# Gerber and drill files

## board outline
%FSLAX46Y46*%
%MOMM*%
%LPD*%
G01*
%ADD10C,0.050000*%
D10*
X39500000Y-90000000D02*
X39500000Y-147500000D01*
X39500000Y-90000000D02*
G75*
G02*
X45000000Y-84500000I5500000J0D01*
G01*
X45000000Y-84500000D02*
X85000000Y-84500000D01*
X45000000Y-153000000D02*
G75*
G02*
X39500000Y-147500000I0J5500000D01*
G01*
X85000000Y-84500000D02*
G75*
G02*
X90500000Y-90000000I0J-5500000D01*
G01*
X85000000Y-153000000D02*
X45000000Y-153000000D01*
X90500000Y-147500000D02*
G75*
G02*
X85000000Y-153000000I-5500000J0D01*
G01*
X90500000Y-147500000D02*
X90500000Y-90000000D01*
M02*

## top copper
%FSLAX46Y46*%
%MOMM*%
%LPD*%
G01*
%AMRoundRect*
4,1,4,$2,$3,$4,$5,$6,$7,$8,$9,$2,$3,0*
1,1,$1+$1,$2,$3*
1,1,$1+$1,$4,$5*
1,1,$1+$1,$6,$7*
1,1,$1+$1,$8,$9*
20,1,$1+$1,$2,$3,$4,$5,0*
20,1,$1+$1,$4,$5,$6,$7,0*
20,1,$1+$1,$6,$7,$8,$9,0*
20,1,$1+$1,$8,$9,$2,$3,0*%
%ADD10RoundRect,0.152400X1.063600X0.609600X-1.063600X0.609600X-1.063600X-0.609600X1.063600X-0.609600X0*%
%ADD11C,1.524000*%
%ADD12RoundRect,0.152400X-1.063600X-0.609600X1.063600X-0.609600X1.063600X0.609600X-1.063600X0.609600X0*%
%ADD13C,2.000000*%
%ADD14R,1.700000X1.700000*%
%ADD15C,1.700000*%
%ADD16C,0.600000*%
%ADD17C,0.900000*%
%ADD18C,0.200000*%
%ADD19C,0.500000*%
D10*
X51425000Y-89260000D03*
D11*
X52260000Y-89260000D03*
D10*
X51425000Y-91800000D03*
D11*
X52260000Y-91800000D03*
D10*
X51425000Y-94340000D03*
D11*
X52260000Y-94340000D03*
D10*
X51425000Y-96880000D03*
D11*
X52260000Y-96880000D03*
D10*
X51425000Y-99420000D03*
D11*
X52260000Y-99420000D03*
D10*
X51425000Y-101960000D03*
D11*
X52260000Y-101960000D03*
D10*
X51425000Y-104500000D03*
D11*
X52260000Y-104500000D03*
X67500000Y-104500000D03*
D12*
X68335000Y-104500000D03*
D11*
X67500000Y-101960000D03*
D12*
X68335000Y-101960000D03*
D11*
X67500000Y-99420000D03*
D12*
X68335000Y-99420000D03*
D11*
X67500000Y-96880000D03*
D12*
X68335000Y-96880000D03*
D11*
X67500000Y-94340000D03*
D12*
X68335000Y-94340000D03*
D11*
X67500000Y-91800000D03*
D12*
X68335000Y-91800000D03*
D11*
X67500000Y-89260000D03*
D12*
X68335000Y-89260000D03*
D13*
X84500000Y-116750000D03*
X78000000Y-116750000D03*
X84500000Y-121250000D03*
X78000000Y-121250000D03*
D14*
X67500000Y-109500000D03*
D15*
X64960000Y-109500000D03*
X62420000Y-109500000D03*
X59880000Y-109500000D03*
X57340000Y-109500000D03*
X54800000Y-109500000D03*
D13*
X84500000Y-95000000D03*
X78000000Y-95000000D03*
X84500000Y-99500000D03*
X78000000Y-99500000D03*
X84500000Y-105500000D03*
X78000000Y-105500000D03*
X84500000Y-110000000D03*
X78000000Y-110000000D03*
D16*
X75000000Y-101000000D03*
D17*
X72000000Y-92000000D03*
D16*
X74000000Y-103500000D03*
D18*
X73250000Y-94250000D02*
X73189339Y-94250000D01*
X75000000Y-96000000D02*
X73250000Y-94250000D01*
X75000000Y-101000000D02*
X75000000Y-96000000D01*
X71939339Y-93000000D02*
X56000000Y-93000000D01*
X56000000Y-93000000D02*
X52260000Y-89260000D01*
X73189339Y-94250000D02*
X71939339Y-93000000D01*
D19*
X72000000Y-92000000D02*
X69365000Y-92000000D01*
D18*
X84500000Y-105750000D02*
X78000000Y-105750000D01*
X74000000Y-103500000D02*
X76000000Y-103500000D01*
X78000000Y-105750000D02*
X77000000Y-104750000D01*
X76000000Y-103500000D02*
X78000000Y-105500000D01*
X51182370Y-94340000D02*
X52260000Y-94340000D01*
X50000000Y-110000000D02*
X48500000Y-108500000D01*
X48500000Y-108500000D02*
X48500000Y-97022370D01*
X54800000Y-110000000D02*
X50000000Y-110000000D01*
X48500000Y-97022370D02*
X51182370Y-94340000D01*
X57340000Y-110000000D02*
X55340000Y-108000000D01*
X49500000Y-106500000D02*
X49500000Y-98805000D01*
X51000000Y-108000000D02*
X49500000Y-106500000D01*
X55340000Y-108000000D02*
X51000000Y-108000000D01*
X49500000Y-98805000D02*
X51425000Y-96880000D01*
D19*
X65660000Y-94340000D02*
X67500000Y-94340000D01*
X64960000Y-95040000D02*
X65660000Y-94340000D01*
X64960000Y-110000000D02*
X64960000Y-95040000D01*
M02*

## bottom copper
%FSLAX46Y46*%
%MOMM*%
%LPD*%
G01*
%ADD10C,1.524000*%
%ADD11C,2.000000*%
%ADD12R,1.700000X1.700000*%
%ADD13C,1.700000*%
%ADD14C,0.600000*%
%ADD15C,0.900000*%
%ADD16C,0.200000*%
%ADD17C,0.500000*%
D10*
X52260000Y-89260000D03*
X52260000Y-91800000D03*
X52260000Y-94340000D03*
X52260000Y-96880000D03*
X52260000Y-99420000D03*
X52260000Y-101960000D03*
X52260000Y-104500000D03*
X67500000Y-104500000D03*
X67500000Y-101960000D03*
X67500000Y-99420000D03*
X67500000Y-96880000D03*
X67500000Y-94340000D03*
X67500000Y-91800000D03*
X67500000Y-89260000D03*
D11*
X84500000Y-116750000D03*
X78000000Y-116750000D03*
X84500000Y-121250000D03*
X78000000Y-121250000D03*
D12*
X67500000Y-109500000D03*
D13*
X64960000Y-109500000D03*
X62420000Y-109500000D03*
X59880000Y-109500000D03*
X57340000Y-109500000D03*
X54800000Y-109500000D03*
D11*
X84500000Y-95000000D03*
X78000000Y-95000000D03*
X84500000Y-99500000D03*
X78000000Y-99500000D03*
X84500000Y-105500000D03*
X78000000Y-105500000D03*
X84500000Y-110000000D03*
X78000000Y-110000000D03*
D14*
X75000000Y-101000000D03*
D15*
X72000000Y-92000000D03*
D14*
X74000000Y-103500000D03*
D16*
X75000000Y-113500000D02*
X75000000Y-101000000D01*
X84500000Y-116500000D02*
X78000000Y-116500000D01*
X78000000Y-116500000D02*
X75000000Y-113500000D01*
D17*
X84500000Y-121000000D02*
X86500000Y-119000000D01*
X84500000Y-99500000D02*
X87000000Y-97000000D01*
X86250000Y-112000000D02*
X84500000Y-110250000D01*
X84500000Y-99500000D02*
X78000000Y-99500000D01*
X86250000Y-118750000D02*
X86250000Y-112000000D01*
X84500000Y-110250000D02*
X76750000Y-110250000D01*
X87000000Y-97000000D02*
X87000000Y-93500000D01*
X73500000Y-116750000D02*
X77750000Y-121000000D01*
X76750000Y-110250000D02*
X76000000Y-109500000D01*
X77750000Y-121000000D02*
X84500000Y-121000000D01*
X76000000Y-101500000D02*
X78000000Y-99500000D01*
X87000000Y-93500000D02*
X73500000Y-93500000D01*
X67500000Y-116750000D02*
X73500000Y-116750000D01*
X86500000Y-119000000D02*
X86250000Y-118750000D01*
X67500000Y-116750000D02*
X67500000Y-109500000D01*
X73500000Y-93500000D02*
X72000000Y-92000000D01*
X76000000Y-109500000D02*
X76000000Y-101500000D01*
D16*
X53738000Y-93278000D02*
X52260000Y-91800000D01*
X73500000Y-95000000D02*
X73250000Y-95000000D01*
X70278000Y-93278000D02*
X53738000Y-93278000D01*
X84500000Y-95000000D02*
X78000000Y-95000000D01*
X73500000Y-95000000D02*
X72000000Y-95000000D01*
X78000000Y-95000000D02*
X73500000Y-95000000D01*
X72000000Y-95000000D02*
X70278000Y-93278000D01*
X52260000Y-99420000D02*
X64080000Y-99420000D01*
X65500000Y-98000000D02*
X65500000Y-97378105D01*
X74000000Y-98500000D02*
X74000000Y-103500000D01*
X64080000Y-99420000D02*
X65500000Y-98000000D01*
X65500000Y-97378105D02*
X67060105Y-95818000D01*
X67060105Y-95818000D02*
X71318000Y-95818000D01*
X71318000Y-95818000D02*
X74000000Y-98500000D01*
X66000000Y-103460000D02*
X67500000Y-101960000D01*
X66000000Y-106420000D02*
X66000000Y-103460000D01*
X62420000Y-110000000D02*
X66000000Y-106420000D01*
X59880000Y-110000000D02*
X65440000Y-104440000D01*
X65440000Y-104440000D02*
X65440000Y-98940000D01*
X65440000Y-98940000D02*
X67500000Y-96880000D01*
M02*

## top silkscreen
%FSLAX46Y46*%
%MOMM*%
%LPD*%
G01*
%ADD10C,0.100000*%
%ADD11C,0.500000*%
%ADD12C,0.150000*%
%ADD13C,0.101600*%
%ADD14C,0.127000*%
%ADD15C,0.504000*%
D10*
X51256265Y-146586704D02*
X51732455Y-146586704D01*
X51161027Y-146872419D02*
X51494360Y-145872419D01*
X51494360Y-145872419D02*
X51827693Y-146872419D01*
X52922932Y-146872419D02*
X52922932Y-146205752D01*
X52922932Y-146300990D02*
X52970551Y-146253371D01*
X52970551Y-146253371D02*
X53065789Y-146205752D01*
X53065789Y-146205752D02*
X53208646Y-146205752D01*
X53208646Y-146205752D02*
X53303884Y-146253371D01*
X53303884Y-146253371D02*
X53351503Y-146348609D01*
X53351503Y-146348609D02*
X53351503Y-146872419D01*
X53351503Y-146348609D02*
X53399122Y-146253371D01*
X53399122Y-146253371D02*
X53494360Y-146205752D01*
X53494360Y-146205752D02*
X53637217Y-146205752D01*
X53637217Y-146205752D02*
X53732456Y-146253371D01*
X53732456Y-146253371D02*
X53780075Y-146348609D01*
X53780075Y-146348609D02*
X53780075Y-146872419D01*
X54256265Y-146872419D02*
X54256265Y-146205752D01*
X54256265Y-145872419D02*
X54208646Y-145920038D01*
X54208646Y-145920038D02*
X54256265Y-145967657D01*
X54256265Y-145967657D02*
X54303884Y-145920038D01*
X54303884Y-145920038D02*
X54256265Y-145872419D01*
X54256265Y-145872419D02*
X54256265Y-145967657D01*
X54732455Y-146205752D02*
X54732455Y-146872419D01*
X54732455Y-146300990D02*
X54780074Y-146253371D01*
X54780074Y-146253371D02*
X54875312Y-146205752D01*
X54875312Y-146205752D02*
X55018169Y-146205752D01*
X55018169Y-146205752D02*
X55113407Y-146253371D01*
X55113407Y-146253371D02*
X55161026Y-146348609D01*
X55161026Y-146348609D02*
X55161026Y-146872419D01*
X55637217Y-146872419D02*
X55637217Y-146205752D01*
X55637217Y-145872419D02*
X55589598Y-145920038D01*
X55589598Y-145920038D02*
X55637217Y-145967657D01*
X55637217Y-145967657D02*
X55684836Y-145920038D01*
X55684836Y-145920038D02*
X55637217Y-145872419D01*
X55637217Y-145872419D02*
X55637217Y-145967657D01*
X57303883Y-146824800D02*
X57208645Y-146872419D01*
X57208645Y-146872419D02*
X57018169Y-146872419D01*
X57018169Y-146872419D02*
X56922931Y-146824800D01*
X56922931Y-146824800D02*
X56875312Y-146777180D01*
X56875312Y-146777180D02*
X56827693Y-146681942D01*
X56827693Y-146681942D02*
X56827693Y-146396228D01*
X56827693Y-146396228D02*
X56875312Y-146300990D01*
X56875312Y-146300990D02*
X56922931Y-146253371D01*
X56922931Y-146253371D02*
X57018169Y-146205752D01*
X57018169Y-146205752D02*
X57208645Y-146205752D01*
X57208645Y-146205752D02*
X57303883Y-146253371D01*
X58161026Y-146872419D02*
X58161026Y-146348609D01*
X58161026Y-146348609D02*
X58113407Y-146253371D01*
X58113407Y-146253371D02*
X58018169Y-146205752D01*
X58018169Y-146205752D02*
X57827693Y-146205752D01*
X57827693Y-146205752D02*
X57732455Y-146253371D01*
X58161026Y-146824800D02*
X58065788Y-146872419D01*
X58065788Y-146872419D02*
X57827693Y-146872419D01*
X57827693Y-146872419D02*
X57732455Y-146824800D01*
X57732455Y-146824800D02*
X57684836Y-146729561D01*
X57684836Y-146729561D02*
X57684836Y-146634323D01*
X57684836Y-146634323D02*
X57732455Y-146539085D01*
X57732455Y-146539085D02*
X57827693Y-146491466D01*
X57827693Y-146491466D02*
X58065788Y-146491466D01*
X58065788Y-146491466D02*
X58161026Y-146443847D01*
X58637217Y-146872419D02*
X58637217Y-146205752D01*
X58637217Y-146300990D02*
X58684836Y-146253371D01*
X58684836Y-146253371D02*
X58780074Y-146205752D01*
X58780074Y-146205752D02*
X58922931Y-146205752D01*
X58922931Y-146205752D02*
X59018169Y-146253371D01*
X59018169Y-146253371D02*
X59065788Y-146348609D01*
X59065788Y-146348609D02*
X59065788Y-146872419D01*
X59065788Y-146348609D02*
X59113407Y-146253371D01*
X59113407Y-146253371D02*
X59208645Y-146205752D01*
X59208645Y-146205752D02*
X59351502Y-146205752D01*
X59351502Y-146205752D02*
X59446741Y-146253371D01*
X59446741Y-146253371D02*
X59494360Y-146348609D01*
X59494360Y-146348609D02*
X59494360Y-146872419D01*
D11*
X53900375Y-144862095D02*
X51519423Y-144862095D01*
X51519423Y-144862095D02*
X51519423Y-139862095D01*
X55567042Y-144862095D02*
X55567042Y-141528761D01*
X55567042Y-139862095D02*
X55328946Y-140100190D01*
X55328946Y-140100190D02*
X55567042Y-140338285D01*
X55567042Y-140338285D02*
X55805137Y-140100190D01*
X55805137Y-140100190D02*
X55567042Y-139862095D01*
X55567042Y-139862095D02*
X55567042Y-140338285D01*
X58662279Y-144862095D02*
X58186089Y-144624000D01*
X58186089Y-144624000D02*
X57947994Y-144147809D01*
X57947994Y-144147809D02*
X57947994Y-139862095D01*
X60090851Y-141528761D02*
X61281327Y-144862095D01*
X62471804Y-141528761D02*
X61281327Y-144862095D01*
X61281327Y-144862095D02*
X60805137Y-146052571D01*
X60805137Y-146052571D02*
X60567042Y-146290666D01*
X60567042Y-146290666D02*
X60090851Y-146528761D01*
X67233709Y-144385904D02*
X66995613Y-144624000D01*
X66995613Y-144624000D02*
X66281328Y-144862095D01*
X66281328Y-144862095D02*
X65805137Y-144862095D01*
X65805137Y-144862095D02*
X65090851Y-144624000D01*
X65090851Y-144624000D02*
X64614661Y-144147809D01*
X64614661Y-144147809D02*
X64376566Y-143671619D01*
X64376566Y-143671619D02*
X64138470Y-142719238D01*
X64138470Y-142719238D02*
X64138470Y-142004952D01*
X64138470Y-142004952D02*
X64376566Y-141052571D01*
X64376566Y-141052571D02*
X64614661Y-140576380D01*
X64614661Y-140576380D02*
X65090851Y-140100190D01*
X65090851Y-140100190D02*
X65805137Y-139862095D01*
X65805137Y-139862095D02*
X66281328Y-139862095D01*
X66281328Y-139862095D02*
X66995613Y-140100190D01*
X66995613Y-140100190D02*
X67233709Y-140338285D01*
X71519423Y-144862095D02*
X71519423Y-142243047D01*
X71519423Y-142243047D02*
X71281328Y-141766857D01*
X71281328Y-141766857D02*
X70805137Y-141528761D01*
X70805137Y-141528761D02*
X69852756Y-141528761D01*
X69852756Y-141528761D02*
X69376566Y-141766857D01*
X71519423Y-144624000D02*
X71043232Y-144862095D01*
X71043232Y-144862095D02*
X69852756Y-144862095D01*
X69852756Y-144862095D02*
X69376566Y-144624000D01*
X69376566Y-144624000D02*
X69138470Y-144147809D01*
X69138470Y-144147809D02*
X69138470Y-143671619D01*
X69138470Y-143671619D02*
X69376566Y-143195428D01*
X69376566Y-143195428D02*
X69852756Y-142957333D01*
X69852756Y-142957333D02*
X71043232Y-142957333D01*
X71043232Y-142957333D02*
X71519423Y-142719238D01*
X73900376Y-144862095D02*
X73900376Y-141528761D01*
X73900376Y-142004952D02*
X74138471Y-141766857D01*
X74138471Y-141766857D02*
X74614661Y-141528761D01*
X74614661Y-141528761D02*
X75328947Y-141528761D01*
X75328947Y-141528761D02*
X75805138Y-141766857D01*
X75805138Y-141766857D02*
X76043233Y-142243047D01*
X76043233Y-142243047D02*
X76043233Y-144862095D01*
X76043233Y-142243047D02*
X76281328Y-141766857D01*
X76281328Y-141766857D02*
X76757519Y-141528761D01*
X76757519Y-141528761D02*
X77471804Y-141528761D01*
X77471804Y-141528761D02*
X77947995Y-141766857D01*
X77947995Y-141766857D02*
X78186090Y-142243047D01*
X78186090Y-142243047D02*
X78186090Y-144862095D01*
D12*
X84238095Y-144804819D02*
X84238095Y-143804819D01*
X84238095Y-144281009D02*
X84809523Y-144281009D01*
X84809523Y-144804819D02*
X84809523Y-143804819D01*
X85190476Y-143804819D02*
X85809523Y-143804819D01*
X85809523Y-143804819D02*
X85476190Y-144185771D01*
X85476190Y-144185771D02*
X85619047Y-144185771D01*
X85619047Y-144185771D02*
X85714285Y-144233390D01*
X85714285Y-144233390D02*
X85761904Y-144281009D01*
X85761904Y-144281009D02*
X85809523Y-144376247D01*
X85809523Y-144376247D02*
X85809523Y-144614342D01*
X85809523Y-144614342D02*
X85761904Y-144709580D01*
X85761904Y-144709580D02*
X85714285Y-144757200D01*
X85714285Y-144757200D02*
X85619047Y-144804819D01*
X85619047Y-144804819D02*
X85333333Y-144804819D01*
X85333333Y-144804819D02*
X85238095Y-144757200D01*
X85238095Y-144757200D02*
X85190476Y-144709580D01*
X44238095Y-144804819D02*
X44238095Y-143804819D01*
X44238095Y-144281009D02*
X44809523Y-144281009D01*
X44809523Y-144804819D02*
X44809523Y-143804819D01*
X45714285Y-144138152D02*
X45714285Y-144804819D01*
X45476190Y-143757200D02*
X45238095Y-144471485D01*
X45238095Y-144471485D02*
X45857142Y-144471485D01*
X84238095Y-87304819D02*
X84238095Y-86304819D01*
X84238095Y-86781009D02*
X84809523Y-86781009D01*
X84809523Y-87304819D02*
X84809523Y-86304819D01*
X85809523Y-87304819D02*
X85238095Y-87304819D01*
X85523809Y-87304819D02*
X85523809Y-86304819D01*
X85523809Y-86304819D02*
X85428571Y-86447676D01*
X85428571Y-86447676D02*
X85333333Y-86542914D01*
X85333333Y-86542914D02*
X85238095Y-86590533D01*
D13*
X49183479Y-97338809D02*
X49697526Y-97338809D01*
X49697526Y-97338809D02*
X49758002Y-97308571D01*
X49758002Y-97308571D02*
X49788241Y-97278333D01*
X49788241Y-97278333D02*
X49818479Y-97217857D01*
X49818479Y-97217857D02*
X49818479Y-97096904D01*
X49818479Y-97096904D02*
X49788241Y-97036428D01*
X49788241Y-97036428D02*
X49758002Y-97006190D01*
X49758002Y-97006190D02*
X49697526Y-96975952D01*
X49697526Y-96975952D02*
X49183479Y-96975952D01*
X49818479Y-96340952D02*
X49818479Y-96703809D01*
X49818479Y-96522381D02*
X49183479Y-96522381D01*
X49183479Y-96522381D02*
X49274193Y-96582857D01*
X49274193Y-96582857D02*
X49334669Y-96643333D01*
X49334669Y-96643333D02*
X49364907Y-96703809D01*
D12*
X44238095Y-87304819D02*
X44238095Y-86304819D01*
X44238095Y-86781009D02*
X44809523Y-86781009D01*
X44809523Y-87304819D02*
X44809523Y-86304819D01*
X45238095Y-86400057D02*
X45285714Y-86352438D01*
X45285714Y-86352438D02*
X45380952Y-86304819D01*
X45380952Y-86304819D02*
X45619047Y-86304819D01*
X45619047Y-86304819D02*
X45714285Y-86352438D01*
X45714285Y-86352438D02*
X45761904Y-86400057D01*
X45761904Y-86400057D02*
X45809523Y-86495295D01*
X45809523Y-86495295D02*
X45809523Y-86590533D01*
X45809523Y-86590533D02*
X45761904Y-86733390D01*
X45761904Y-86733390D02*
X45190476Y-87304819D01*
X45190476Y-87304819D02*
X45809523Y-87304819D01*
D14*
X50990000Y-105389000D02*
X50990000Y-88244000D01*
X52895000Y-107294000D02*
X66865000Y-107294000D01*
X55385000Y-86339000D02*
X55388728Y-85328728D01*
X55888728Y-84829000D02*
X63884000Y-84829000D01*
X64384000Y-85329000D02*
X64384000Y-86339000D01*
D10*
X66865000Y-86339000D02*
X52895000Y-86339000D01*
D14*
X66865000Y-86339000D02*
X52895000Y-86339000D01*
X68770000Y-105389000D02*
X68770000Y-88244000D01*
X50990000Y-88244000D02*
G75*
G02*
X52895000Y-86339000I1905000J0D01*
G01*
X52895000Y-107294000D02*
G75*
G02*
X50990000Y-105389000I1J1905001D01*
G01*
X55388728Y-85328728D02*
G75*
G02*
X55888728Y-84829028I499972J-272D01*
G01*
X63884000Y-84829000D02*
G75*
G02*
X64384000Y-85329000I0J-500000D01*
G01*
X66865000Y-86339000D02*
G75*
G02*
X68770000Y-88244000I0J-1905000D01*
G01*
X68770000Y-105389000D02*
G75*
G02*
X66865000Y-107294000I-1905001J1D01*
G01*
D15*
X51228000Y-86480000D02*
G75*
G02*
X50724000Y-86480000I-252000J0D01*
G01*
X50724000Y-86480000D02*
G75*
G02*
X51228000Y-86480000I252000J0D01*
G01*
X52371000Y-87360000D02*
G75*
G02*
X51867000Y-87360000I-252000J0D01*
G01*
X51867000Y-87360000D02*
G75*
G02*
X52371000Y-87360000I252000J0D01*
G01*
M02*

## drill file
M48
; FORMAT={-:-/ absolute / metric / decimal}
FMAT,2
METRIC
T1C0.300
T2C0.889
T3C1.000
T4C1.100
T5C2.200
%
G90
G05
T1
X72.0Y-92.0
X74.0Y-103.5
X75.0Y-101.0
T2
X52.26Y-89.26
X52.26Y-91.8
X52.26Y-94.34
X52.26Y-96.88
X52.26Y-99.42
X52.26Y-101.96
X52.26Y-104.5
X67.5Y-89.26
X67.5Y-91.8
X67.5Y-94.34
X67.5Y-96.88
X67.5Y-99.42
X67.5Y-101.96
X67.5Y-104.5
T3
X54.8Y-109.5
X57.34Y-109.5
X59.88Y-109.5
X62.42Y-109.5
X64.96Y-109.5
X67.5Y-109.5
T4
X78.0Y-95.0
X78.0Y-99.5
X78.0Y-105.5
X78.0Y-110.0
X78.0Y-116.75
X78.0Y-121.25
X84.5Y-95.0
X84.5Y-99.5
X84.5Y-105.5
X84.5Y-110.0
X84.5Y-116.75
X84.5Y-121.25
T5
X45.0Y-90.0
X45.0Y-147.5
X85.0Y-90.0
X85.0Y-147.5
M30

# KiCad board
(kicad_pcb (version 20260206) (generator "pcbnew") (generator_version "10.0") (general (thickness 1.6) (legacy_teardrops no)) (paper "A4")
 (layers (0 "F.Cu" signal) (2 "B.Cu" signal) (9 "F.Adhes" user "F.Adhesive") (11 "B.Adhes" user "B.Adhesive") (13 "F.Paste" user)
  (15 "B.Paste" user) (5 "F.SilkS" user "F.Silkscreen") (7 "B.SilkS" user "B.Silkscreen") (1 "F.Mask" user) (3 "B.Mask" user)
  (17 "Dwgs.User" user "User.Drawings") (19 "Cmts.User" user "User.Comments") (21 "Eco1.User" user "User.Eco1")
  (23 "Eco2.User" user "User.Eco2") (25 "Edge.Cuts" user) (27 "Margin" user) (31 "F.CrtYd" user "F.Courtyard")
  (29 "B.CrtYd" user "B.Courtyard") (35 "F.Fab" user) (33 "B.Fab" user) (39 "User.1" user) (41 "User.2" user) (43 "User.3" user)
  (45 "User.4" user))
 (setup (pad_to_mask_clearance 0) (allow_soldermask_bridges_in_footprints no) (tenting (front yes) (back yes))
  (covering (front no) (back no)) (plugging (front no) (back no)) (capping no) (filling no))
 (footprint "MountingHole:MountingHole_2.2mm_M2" (layer "F.Cu") (at 85 147.5)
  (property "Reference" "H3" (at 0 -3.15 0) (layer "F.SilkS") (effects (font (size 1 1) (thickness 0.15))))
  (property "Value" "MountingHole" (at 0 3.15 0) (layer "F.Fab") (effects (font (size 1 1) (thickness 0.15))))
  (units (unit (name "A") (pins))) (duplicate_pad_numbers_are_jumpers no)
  (pad "" np_thru_hole circle (at 0 0) (size 2.2 2.2) (drill 2.2) (layers "*.Cu" "*.Mask")))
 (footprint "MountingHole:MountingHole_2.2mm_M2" (layer "F.Cu") (at 45 147.5)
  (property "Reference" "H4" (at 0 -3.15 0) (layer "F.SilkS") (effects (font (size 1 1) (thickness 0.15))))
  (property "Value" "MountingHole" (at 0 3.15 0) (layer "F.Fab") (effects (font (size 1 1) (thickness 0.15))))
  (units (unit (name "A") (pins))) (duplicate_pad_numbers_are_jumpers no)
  (pad "" np_thru_hole circle (at 0 0) (size 2.2 2.2) (drill 2.2) (layers "*.Cu" "*.Mask")))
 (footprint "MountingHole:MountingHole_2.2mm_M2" (layer "F.Cu") (at 85 90)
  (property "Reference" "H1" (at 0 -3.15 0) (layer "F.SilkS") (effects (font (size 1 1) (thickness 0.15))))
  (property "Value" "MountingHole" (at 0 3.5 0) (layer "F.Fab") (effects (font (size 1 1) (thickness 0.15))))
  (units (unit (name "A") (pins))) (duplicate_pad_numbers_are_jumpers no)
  (pad "" np_thru_hole circle (at 0 0) (size 2.2 2.2) (drill 2.2) (layers "*.Cu" "*.Mask")))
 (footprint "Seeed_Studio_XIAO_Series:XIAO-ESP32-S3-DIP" (layer "F.Cu") (at 59.88 96.88 90)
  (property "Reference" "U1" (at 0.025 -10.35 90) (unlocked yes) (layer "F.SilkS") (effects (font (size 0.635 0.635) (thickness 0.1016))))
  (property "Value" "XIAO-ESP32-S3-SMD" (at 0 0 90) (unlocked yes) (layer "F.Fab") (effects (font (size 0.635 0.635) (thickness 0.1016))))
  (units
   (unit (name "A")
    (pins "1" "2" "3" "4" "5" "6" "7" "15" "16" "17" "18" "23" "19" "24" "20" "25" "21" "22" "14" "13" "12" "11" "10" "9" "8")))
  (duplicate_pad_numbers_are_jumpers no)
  (fp_line (start -8.509 -8.89) (end 8.636 -8.89) (stroke (width 0.127) (type solid)) (layer "F.SilkS"))
  (fp_line (start -10.414 -6.985) (end -10.414 6.985) (stroke (width 0.127) (type solid)) (layer "F.SilkS"))
  (fp_line (start 10.541 -4.495) (end 11.551272 -4.491272) (stroke (width 0.127) (type solid)) (layer "F.SilkS"))
  (fp_line (start 12.051 -3.991272) (end 12.051 4.004) (stroke (width 0.127) (type solid)) (layer "F.SilkS"))
  (fp_line (start 11.551 4.504) (end 10.541 4.504) (stroke (width 0.127) (type solid)) (layer "F.SilkS"))
  (fp_line (start 10.541 6.985) (end 10.541 -6.985) (stroke (width 0.1) (type solid)) (layer "F.SilkS"))
  (fp_line (start 10.541 6.985) (end 10.541 -6.985) (stroke (width 0.127) (type solid)) (layer "F.SilkS"))
  (fp_line (start -8.509 8.89) (end 8.636 8.89) (stroke (width 0.127) (type solid)) (layer "F.SilkS"))
  (fp_arc (start 8.636 -8.89) (mid 9.983038 -8.332038) (end 10.541 -6.985) (stroke (width 0.127) (type solid)) (layer "F.SilkS"))
  (fp_arc (start -10.414 -6.985) (mid -9.856038 -8.332038) (end -8.509 -8.89) (stroke (width 0.127) (type solid)) (layer "F.SilkS"))
  (fp_arc (start 11.551272 -4.491272) (mid 11.904644 -4.344724) (end 12.051 -3.991272) (stroke (width 0.127) (type default))
   (layer "F.SilkS"))
  (fp_arc (start 12.051 4.004) (mid 11.904553 4.357553) (end 11.551 4.504) (stroke (width 0.127) (type default)) (layer "F.SilkS"))
  (fp_arc (start 10.541 6.985) (mid 9.983038 8.332038) (end 8.636 8.89) (stroke (width 0.127) (type solid)) (layer "F.SilkS"))
  (fp_arc (start -8.509 8.89) (mid -9.856038 8.332038) (end -10.414 6.985) (stroke (width 0.127) (type solid)) (layer "F.SilkS"))
  (fp_circle (center 10.4 -8.904) (end 10.654 -8.904) (stroke (width 0.5) (type solid)) (fill yes) (layer "F.SilkS"))
  (fp_circle (center 9.52 -7.761) (end 9.774 -7.761) (stroke (width 0.5) (type solid)) (fill yes) (layer "F.SilkS"))
  (pad "1" smd roundrect (at 7.62 -8.455 180) (size 2.432 1.524) (layers "F.Cu" "F.Mask") (roundrect_rratio 0.1) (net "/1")
   (thermal_bridge_angle 45))
  (pad "1" thru_hole circle (at 7.62 -7.62 180) (size 1.524 1.524) (drill 0.889) (layers "*.Cu" "*.Mask") (remove_unused_layers no)
   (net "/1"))
  (pad "2" smd roundrect (at 5.08 -8.455 180) (size 2.432 1.524) (layers "F.Cu" "F.Mask") (roundrect_rratio 0.1) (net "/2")
   (thermal_bridge_angle 45))
  (pad "2" thru_hole circle (at 5.08 -7.62 180) (size 1.524 1.524) (drill 0.889) (layers "*.Cu" "*.Mask") (remove_unused_layers no)
   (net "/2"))
  (pad "3" smd roundrect (at 2.54 -8.455 180) (size 2.432 1.524) (layers "F.Cu" "F.Mask") (roundrect_rratio 0.1) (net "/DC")
   (thermal_bridge_angle 45))
  (pad "3" thru_hole circle (at 2.54 -7.62 180) (size 1.524 1.524) (drill 0.889) (layers "*.Cu" "*.Mask") (remove_unused_layers no)
   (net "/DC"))
  (pad "4" smd roundrect (at 0 -8.455 180) (size 2.432 1.524) (layers "F.Cu" "F.Mask") (roundrect_rratio 0.1) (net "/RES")
   (thermal_bridge_angle 45))
  (pad "4" thru_hole circle (at 0 -7.62 180) (size 1.524 1.524) (drill 0.889) (layers "*.Cu" "*.Mask") (remove_unused_layers no)
   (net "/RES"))
  (pad "5" smd roundrect (at -2.54 -8.455 180) (size 2.432 1.524) (layers "F.Cu" "F.Mask") (roundrect_rratio 0.1) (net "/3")
   (thermal_bridge_angle 45))
  (pad "5" thru_hole circle (at -2.54 -7.62 180) (size 1.524 1.524) (drill 0.889) (layers "*.Cu" "*.Mask") (remove_unused_layers no)
   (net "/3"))
  (pad "6" smd roundrect (at -5.08 -8.455 180) (size 2.432 1.524) (layers "F.Cu" "F.Mask") (roundrect_rratio 0.1)
   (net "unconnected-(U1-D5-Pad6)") (thermal_bridge_angle 45))
  (pad "6" thru_hole circle (at -5.08 -7.62 180) (size 1.524 1.524) (drill 0.889) (layers "*.Cu" "*.Mask") (remove_unused_layers no)
   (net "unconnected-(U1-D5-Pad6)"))
  (pad "7" smd roundrect (at -7.62 -8.455 180) (size 2.432 1.524) (layers "F.Cu" "F.Mask") (roundrect_rratio 0.1)
   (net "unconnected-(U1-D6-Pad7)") (thermal_bridge_angle 45))
  (pad "7" thru_hole circle (at -7.62 -7.62 180) (size 1.524 1.524) (drill 0.889) (layers "*.Cu" "*.Mask") (remove_unused_layers no)
   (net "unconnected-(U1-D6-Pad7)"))
  (pad "8" thru_hole circle (at -7.62 7.62) (size 1.524 1.524) (drill 0.889) (layers "*.Cu" "*.Mask") (remove_unused_layers no)
   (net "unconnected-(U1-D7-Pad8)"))
  (pad "8" smd roundrect (at -7.62 8.455) (size 2.432 1.524) (layers "F.Cu" "F.Mask") (roundrect_rratio 0.1)
   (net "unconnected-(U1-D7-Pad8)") (thermal_bridge_angle 45))
  (pad "9" thru_hole circle (at -5.08 7.62) (size 1.524 1.524) (drill 0.889) (layers "*.Cu" "*.Mask") (remove_unused_layers no) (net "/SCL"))
  (pad "9" smd roundrect (at -5.08 8.455) (size 2.432 1.524) (layers "F.Cu" "F.Mask") (roundrect_rratio 0.1) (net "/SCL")
   (thermal_bridge_angle 45))
  (pad "10" thru_hole circle (at -2.54 7.62) (size 1.524 1.524) (drill 0.889) (layers "*.Cu" "*.Mask") (remove_unused_layers no)
   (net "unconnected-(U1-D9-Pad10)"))
  (pad "10" smd roundrect (at -2.54 8.455) (size 2.432 1.524) (layers "F.Cu" "F.Mask") (roundrect_rratio 0.1)
   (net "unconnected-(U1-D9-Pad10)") (thermal_bridge_angle 45))
  (pad "11" thru_hole circle (at 0 7.62) (size 1.524 1.524) (drill 0.889) (layers "*.Cu" "*.Mask") (remove_unused_layers no) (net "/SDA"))
  (pad "11" smd roundrect (at 0 8.455) (size 2.432 1.524) (layers "F.Cu" "F.Mask") (roundrect_rratio 0.1) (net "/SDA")
   (thermal_bridge_angle 45))
  (pad "12" thru_hole circle (at 2.54 7.62) (size 1.524 1.524) (drill 0.889) (layers "*.Cu" "*.Mask") (remove_unused_layers no)
   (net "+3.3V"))
  (pad "12" smd roundrect (at 2.54 8.455) (size 2.432 1.524) (layers "F.Cu" "F.Mask") (roundrect_rratio 0.1) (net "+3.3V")
   (thermal_bridge_angle 45))
  (pad "13" thru_hole circle (at 5.08 7.62) (size 1.524 1.524) (drill 0.889) (layers "*.Cu" "*.Mask") (remove_unused_layers no) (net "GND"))
  (pad "13" smd roundrect (at 5.08 8.455) (size 2.432 1.524) (layers "F.Cu" "F.Mask") (roundrect_rratio 0.1) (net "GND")
   (thermal_bridge_angle 45))
  (pad "14" thru_hole circle (at 7.62 7.62) (size 1.524 1.524) (drill 0.889) (layers "*.Cu" "*.Mask") (remove_unused_layers no)
   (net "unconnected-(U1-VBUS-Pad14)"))
  (pad "14" smd roundrect (at 7.62 8.455) (size 2.432 1.524) (layers "F.Cu" "F.Mask") (roundrect_rratio 0.1)
   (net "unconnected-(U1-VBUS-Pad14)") (thermal_bridge_angle 45)))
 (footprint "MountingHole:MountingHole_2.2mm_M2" (layer "F.Cu") (at 45 90)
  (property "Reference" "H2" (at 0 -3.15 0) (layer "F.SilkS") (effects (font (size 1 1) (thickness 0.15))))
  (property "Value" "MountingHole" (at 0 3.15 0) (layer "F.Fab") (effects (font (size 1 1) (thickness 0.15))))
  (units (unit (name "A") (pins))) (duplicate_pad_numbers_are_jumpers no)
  (pad "" np_thru_hole circle (at 0 0) (size 2.2 2.2) (drill 2.2) (layers "*.Cu" "*.Mask")))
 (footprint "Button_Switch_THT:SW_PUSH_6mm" (layer "B.Cu") (at 84.5 116.75 180)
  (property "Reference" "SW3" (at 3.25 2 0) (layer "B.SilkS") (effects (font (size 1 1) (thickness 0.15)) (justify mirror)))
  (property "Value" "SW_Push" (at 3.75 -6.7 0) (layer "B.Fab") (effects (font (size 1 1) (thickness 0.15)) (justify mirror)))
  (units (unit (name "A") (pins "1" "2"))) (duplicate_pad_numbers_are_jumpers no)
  (pad "1" thru_hole circle (at 0 0 90) (size 2 2) (drill 1.1) (layers "*.Cu" "*.Mask") (remove_unused_layers no) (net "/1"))
  (pad "1" thru_hole circle (at 6.5 0 90) (size 2 2) (drill 1.1) (layers "*.Cu" "*.Mask") (remove_unused_layers no) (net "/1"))
  (pad "2" thru_hole circle (at 0 -4.5 90) (size 2 2) (drill 1.1) (layers "*.Cu" "*.Mask") (remove_unused_layers no) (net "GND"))
  (pad "2" thru_hole circle (at 6.5 -4.5 90) (size 2 2) (drill 1.1) (layers "*.Cu" "*.Mask") (remove_unused_layers no) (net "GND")))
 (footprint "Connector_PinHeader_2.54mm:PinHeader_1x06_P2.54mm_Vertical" (layer "B.Cu") (at 67.5 109.5 90)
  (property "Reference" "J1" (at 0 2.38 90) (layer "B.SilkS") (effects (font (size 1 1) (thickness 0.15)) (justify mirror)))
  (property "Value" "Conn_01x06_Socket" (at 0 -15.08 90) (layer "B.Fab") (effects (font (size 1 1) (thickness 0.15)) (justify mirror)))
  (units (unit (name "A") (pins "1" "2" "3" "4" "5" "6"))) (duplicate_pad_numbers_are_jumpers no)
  (pad "1" thru_hole rect (at 0 0 90) (size 1.7 1.7) (drill 1) (layers "*.Cu" "*.Mask") (remove_unused_layers no) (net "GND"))
  (pad "2" thru_hole circle (at 0 -2.54 90) (size 1.7 1.7) (drill 1) (layers "*.Cu" "*.Mask") (remove_unused_layers no) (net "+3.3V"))
  (pad "3" thru_hole circle (at 0 -5.08 90) (size 1.7 1.7) (drill 1) (layers "*.Cu" "*.Mask") (remove_unused_layers no) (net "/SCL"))
  (pad "4" thru_hole circle (at 0 -7.62 90) (size 1.7 1.7) (drill 1) (layers "*.Cu" "*.Mask") (remove_unused_layers no) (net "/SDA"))
  (pad "5" thru_hole circle (at 0 -10.16 90) (size 1.7 1.7) (drill 1) (layers "*.Cu" "*.Mask") (remove_unused_layers no) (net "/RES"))
  (pad "6" thru_hole circle (at 0 -12.7 90) (size 1.7 1.7) (drill 1) (layers "*.Cu" "*.Mask") (remove_unused_layers no) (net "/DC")))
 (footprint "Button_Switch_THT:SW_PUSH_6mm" (layer "B.Cu") (at 84.5 95 180)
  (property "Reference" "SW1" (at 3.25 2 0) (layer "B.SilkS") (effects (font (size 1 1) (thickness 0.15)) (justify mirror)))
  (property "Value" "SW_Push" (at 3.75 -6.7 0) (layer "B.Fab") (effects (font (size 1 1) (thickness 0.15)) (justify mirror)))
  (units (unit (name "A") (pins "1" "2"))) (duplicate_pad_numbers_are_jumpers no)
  (pad "1" thru_hole circle (at 0 0 90) (size 2 2) (drill 1.1) (layers "*.Cu" "*.Mask") (remove_unused_layers no) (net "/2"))
  (pad "1" thru_hole circle (at 6.5 0 90) (size 2 2) (drill 1.1) (layers "*.Cu" "*.Mask") (remove_unused_layers no) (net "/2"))
  (pad "2" thru_hole circle (at 0 -4.5 90) (size 2 2) (drill 1.1) (layers "*.Cu" "*.Mask") (remove_unused_layers no) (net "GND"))
  (pad "2" thru_hole circle (at 6.5 -4.5 90) (size 2 2) (drill 1.1) (layers "*.Cu" "*.Mask") (remove_unused_layers no) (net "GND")))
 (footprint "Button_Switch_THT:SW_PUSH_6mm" (layer "B.Cu") (at 84.5 105.5 180)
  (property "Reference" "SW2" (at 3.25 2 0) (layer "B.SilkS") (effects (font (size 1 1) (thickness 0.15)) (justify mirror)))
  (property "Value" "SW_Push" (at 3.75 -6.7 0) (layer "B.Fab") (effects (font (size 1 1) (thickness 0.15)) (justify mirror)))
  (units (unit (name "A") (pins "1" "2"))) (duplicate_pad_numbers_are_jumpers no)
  (pad "1" thru_hole circle (at 0 0 90) (size 2 2) (drill 1.1) (layers "*.Cu" "*.Mask") (remove_unused_layers no) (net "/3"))
  (pad "1" thru_hole circle (at 6.5 0 90) (size 2 2) (drill 1.1) (layers "*.Cu" "*.Mask") (remove_unused_layers no) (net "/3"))
  (pad "2" thru_hole circle (at 0 -4.5 90) (size 2 2) (drill 1.1) (layers "*.Cu" "*.Mask") (remove_unused_layers no) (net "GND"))
  (pad "2" thru_hole circle (at 6.5 -4.5 90) (size 2 2) (drill 1.1) (layers "*.Cu" "*.Mask") (remove_unused_layers no) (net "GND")))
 (gr_line (start 39.5 90) (end 39.5 147.5) (stroke (width 0.05) (type default)) (layer "Edge.Cuts"))
 (gr_arc (start 39.5 90) (mid 41.110913 86.110913) (end 45 84.5) (stroke (width 0.05) (type default)) (layer "Edge.Cuts"))
 (gr_line (start 45 84.5) (end 85 84.5) (stroke (width 0.05) (type default)) (layer "Edge.Cuts"))
 (gr_arc (start 45 153) (mid 41.110913 151.389087) (end 39.5 147.5) (stroke (width 0.05) (type default)) (layer "Edge.Cuts"))
 (gr_arc (start 85 84.5) (mid 88.889087 86.110913) (end 90.5 90) (stroke (width 0.05) (type default)) (layer "Edge.Cuts"))
 (gr_line (start 85 153) (end 45 153) (stroke (width 0.05) (type default)) (layer "Edge.Cuts"))
 (gr_arc (start 90.5 147.5) (mid 88.889087 151.389087) (end 85 153) (stroke (width 0.05) (type default)) (layer "Edge.Cuts"))
 (gr_line (start 90.5 147.5) (end 90.5 90) (stroke (width 0.05) (type default)) (layer "Edge.Cuts"))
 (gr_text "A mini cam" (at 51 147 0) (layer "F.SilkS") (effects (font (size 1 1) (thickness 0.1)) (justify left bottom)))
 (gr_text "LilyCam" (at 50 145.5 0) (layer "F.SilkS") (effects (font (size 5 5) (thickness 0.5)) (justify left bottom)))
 (segment (start 73.25 94.25) (end 73.189339 94.25) (width 0.2) (layer "F.Cu") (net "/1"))
 (segment (start 75 96) (end 73.25 94.25) (width 0.2) (layer "F.Cu") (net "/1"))
 (segment (start 75 101) (end 75 96) (width 0.2) (layer "F.Cu") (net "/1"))
 (segment (start 71.939339 93) (end 56 93) (width 0.2) (layer "F.Cu") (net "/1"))
 (segment (start 56 93) (end 52.26 89.26) (width 0.2) (layer "F.Cu") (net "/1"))
 (segment (start 73.189339 94.25) (end 71.939339 93) (width 0.2) (layer "F.Cu") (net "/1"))
 (via (at 75 101) (size 0.6) (drill 0.3) (layers "F.Cu" "B.Cu") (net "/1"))
 (segment (start 75 113.5) (end 75 101) (width 0.2) (layer "B.Cu") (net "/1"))
 (segment (start 84.5 116.5) (end 78 116.5) (width 0.2) (layer "B.Cu") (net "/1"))
 (segment (start 78 116.5) (end 75 113.5) (width 0.2) (layer "B.Cu") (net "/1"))
 (segment (start 72 92) (end 69.365 92) (width 0.5) (layer "F.Cu") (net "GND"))
 (via (at 72 92) (size 0.9) (drill 0.3) (layers "F.Cu" "B.Cu") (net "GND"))
 (segment (start 84.5 121) (end 86.5 119) (width 0.5) (layer "B.Cu") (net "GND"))
 (segment (start 84.5 99.5) (end 87 97) (width 0.5) (layer "B.Cu") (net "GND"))
 (segment (start 86.25 112) (end 84.5 110.25) (width 0.5) (layer "B.Cu") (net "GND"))
 (segment (start 84.5 99.5) (end 78 99.5) (width 0.5) (layer "B.Cu") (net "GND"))
 (segment (start 86.25 118.75) (end 86.25 112) (width 0.5) (layer "B.Cu") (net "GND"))
 (segment (start 84.5 110.25) (end 76.75 110.25) (width 0.5) (layer "B.Cu") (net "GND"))
 (segment (start 87 97) (end 87 93.5) (width 0.5) (layer "B.Cu") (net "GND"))
 (segment (start 73.5 116.75) (end 77.75 121) (width 0.5) (layer "B.Cu") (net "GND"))
 (segment (start 76.75 110.25) (end 76 109.5) (width 0.5) (layer "B.Cu") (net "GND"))
 (segment (start 77.75 121) (end 84.5 121) (width 0.5) (layer "B.Cu") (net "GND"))
 (segment (start 76 101.5) (end 78 99.5) (width 0.5) (layer "B.Cu") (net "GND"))
 (segment (start 87 93.5) (end 73.5 93.5) (width 0.5) (layer "B.Cu") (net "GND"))
 (segment (start 67.5 116.75) (end 73.5 116.75) (width 0.5) (layer "B.Cu") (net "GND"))
 (segment (start 86.5 119) (end 86.25 118.75) (width 0.5) (layer "B.Cu") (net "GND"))
 (segment (start 67.5 116.75) (end 67.5 109.5) (width 0.5) (layer "B.Cu") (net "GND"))
 (segment (start 73.5 93.5) (end 72 92) (width 0.5) (layer "B.Cu") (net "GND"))
 (segment (start 76 109.5) (end 76 101.5) (width 0.5) (layer "B.Cu") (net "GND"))
 (segment (start 53.738 93.278) (end 52.26 91.8) (width 0.2) (layer "B.Cu") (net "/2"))
 (segment (start 73.5 95) (end 73.25 95) (width 0.2) (layer "B.Cu") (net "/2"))
 (segment (start 70.278 93.278) (end 53.738 93.278) (width 0.2) (layer "B.Cu") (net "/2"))
 (segment (start 84.5 95) (end 78 95) (width 0.2) (layer "B.Cu") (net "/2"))
 (segment (start 73.5 95) (end 72 95) (width 0.2) (layer "B.Cu") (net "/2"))
 (segment (start 78 95) (end 73.5 95) (width 0.2) (layer "B.Cu") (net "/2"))
 (segment (start 72 95) (end 70.278 93.278) (width 0.2) (layer "B.Cu") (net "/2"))
 (segment (start 84.5 105.75) (end 78 105.75) (width 0.2) (layer "F.Cu") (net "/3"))
 (segment (start 74 103.5) (end 76 103.5) (width 0.2) (layer "F.Cu") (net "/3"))
 (segment (start 78 105.75) (end 77 104.75) (width 0.2) (layer "F.Cu") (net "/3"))
 (segment (start 76 103.5) (end 78 105.5) (width 0.2) (layer "F.Cu") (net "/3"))
 (via (at 74 103.5) (size 0.6) (drill 0.3) (layers "F.Cu" "B.Cu") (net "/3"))
 (segment (start 52.26 99.42) (end 64.08 99.42) (width 0.2) (layer "B.Cu") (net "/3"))
 (segment (start 65.5 98) (end 65.5 97.378105) (width 0.2) (layer "B.Cu") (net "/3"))
 (segment (start 74 98.5) (end 74 103.5) (width 0.2) (layer "B.Cu") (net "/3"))
 (segment (start 64.08 99.42) (end 65.5 98) (width 0.2) (layer "B.Cu") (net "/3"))
 (segment (start 65.5 97.378105) (end 67.060105 95.818) (width 0.2) (layer "B.Cu") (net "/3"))
 (segment (start 67.060105 95.818) (end 71.318 95.818) (width 0.2) (layer "B.Cu") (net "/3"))
 (segment (start 71.318 95.818) (end 74 98.5) (width 0.2) (layer "B.Cu") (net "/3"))
 (segment (start 51.18237 94.34) (end 52.26 94.34) (width 0.2) (layer "F.Cu") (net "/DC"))
 (segment (start 50 110) (end 48.5 108.5) (width 0.2) (layer "F.Cu") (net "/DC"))
 (segment (start 48.5 108.5) (end 48.5 97.02237) (width 0.2) (layer "F.Cu") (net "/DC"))
 (segment (start 54.8 110) (end 50 110) (width 0.2) (layer "F.Cu") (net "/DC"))
 (segment (start 48.5 97.02237) (end 51.18237 94.34) (width 0.2) (layer "F.Cu") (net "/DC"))
 (segment (start 57.34 110) (end 55.34 108) (width 0.2) (layer "F.Cu") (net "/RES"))
 (segment (start 49.5 106.5) (end 49.5 98.805) (width 0.2) (layer "F.Cu") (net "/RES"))
 (segment (start 51 108) (end 49.5 106.5) (width 0.2) (layer "F.Cu") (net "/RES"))
 (segment (start 55.34 108) (end 51 108) (width 0.2) (layer "F.Cu") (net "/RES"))
 (segment (start 49.5 98.805) (end 51.425 96.88) (width 0.2) (layer "F.Cu") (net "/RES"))
 (segment (start 66 103.46) (end 67.5 101.96) (width 0.2) (layer "B.Cu") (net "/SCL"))
 (segment (start 66 106.42) (end 66 103.46) (width 0.2) (layer "B.Cu") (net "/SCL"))
 (segment (start 62.42 110) (end 66 106.42) (width 0.2) (layer "B.Cu") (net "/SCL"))
 (segment (start 59.88 110) (end 65.44 104.44) (width 0.2) (layer "B.Cu") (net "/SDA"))
 (segment (start 65.44 104.44) (end 65.44 98.94) (width 0.2) (layer "B.Cu") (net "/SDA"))
 (segment (start 65.44 98.94) (end 67.5 96.88) (width 0.2) (layer "B.Cu") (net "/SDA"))
 (segment (start 65.66 94.34) (end 67.5 94.34) (width 0.5) (layer "F.Cu") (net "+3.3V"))
 (segment (start 64.96 95.04) (end 65.66 94.34) (width 0.5) (layer "F.Cu") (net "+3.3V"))
 (segment (start 64.96 110) (end 64.96 95.04) (width 0.5) (layer "F.Cu") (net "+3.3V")))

